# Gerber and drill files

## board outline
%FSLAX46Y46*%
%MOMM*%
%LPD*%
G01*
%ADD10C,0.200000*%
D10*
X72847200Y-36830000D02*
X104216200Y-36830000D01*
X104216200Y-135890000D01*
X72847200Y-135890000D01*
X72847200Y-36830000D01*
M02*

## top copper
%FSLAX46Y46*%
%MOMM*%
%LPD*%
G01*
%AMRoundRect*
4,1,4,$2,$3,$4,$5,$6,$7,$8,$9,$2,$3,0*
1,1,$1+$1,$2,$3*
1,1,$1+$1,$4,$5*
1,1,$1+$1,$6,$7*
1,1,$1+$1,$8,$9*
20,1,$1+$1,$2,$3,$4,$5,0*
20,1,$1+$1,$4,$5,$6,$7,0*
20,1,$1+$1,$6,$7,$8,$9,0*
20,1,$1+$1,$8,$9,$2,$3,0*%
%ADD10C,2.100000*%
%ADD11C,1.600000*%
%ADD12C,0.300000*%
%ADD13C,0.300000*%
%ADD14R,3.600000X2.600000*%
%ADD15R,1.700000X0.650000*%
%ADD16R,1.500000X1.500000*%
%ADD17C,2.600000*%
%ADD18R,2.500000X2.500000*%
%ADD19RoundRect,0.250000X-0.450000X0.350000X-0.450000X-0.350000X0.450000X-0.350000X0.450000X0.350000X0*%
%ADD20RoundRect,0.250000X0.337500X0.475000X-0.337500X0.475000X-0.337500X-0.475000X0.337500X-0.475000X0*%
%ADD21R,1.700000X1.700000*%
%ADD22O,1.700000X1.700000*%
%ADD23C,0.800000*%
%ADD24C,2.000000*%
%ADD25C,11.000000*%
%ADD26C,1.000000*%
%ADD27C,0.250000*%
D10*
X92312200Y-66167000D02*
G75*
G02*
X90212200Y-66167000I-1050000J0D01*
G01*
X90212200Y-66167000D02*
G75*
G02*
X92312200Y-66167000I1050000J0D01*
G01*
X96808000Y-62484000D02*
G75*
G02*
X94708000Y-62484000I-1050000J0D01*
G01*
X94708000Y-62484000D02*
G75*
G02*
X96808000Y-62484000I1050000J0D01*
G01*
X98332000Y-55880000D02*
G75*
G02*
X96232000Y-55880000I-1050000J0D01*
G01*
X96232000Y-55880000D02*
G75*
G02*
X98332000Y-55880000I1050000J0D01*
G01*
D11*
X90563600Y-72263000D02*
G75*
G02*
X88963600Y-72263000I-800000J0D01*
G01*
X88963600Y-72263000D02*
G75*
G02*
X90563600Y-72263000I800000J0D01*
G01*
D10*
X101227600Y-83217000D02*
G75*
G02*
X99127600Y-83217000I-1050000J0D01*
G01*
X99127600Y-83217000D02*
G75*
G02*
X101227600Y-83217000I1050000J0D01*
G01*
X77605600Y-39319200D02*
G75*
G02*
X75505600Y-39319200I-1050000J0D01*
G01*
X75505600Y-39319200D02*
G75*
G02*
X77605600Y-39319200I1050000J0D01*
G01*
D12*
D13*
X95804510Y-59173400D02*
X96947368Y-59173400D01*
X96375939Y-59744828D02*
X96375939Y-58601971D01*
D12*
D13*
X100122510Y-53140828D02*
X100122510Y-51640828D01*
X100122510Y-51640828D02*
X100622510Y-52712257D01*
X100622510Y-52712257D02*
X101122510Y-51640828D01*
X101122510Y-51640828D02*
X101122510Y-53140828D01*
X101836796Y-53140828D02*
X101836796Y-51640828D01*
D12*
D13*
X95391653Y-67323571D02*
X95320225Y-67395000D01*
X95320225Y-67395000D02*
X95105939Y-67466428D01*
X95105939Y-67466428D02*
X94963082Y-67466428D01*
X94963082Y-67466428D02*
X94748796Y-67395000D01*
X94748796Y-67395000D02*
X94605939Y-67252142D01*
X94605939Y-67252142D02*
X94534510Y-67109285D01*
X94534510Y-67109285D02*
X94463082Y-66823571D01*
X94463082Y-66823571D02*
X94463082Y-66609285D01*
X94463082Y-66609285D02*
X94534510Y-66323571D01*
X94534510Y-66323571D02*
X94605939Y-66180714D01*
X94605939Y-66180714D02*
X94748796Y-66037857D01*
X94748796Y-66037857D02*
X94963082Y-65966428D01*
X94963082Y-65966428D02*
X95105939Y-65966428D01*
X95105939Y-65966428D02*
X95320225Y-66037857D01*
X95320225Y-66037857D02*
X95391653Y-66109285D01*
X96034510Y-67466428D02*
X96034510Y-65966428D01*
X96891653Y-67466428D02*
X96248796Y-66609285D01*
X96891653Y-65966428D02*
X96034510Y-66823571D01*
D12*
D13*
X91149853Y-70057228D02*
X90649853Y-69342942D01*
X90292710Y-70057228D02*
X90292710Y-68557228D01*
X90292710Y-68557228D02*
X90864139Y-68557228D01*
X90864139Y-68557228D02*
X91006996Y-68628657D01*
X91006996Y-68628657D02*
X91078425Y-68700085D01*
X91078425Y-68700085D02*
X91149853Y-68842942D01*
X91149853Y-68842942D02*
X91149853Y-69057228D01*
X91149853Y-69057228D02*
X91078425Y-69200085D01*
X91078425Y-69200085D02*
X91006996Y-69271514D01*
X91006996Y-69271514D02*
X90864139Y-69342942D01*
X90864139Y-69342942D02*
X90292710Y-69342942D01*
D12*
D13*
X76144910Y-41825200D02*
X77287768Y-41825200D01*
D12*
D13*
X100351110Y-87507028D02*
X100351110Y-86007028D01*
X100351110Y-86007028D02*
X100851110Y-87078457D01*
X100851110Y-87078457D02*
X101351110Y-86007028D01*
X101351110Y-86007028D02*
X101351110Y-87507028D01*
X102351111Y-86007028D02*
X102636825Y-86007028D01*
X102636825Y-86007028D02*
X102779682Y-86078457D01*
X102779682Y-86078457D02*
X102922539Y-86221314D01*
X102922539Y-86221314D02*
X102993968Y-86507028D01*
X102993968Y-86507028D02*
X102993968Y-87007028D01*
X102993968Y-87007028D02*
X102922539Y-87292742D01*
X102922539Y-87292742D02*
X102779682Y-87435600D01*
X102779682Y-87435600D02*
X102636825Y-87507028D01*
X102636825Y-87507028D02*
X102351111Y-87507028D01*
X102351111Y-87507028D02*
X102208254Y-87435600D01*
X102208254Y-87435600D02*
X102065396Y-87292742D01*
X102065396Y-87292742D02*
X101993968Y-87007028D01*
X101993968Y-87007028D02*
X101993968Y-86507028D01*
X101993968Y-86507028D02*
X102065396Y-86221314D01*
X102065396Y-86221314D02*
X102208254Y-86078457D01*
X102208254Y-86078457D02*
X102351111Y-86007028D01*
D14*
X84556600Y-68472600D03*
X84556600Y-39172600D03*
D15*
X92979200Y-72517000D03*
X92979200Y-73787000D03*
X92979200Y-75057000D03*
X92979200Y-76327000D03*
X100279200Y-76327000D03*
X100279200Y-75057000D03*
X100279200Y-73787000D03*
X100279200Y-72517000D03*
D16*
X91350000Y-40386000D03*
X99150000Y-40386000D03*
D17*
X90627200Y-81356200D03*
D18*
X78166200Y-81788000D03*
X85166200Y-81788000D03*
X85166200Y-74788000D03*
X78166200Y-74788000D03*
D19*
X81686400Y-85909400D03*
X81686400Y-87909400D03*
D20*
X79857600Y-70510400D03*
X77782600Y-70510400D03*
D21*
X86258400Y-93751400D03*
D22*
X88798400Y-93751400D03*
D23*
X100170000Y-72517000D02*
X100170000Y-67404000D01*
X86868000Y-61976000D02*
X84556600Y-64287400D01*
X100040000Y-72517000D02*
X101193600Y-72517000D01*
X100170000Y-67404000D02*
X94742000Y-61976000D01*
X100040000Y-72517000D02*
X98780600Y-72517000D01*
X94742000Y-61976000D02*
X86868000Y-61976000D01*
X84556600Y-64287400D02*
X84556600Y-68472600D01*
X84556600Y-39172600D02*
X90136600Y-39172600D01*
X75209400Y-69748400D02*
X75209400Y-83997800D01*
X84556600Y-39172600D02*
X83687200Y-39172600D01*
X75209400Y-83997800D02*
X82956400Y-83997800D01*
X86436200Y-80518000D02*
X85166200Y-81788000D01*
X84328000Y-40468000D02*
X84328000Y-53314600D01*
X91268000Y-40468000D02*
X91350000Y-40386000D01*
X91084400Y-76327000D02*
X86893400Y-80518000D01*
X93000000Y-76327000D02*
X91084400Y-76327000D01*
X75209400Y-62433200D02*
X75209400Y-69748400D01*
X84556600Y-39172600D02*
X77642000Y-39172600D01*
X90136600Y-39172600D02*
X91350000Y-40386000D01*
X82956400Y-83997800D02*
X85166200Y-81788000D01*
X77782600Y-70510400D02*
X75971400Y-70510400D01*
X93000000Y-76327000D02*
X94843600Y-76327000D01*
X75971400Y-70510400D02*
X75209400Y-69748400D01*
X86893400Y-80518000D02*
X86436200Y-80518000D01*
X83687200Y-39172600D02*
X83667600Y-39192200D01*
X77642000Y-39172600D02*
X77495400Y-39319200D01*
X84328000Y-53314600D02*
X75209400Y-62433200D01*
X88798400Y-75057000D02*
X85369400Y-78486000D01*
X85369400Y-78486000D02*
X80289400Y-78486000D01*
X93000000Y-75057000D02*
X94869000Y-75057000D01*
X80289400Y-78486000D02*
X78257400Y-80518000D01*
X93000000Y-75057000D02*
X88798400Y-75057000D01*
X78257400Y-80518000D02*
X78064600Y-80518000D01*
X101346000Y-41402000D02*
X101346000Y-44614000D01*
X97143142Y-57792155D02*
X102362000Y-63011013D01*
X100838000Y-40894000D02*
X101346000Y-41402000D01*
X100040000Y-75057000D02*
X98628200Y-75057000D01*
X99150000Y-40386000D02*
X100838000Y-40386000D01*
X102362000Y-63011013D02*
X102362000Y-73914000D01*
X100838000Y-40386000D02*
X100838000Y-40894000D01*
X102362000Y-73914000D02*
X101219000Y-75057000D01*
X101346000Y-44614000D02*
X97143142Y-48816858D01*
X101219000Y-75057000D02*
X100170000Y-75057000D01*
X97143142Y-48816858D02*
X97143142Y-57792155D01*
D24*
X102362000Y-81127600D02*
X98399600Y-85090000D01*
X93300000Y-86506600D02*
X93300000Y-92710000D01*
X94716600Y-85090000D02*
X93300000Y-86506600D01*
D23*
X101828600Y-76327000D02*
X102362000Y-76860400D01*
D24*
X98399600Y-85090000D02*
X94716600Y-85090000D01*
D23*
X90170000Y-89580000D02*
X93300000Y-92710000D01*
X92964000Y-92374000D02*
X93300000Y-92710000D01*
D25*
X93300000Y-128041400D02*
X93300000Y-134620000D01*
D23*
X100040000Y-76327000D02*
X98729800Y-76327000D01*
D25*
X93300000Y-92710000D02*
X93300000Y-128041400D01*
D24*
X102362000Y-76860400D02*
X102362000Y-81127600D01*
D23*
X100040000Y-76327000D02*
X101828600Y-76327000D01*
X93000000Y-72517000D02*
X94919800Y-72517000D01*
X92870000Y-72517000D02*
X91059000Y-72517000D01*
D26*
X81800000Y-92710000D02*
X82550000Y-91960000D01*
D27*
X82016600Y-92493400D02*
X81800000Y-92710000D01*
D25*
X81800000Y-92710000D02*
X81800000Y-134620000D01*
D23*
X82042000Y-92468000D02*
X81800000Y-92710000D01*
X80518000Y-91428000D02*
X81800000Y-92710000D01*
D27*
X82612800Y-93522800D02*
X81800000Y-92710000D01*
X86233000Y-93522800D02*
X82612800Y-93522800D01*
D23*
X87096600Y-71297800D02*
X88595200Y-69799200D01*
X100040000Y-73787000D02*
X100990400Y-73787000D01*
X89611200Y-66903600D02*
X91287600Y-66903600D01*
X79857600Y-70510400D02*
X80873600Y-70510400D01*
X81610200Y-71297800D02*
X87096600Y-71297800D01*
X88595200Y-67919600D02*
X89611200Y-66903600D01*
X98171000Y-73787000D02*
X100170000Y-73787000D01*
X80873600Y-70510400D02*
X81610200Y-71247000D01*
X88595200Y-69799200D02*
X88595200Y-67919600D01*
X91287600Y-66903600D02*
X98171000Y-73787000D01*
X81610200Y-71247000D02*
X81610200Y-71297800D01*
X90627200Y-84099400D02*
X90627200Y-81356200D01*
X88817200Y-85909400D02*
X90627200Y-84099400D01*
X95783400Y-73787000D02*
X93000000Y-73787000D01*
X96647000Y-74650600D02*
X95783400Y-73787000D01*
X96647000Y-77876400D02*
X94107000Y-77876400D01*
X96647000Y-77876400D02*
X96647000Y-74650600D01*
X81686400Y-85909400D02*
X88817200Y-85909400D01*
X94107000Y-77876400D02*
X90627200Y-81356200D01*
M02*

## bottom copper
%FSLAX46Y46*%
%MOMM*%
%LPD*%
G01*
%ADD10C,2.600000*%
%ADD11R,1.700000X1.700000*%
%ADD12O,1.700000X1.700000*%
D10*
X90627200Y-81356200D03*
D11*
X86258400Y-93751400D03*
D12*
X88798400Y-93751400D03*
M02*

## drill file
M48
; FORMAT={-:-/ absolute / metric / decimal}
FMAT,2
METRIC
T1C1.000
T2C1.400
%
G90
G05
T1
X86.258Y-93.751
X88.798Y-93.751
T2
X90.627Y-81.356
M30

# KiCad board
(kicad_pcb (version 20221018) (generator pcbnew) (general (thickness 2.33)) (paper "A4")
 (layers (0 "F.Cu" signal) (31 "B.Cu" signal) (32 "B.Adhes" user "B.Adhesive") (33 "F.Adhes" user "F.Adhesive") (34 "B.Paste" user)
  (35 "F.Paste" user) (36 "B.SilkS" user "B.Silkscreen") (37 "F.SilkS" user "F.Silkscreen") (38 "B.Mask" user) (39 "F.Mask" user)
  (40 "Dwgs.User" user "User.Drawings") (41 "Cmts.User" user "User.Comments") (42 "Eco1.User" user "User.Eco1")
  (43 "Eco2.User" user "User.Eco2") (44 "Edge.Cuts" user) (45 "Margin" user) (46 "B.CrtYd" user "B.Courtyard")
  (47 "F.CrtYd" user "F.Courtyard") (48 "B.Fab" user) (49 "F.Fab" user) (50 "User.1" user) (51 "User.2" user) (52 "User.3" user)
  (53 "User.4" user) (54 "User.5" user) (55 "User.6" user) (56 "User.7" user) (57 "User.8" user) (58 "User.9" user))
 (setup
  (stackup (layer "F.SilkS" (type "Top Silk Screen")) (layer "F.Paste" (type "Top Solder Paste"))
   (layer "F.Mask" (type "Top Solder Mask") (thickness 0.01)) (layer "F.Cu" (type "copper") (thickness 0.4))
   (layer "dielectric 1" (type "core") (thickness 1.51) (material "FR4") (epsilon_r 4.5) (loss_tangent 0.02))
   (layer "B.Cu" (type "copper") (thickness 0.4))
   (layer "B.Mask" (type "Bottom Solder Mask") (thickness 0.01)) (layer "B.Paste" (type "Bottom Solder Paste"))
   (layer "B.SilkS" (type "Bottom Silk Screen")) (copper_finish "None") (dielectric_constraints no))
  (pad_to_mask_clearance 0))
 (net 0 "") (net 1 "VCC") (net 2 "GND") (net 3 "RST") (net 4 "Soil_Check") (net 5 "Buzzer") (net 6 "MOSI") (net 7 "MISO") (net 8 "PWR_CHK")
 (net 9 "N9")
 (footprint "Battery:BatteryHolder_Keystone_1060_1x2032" (layer "F.Cu") (at 84.5566 53.8226 90)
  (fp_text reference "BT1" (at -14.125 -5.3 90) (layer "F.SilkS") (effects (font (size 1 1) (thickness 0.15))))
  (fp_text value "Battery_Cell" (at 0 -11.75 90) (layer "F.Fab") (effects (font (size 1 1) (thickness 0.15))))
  (pad "1" smd rect (at -14.65 0 270) (size 2.6 3.6) (layers "F.Cu" "F.Paste" "F.Mask") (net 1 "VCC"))
  (pad "2" smd rect (at 14.65 0 270) (size 2.6 3.6) (layers "F.Cu" "F.Paste" "F.Mask") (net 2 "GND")))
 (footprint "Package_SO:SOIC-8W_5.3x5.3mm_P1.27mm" (layer "F.Cu") (at 96.6292 74.422)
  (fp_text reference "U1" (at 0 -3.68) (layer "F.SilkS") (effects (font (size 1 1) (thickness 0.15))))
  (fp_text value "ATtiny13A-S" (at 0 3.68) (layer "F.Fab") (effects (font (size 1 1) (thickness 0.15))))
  (pad "1" smd rect (at -3.65 -1.905) (size 1.7 0.65) (layers "F.Cu" "F.Paste" "F.Mask") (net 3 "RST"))
  (pad "2" smd rect (at -3.65 -0.635) (size 1.7 0.65) (layers "F.Cu" "F.Paste" "F.Mask") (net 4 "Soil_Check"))
  (pad "3" smd rect (at -3.65 0.635) (size 1.7 0.65) (layers "F.Cu" "F.Paste" "F.Mask") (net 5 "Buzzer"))
  (pad "4" smd rect (at -3.65 1.905) (size 1.7 0.65) (layers "F.Cu" "F.Paste" "F.Mask") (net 2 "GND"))
  (pad "5" smd rect (at 3.65 1.905) (size 1.7 0.65) (layers "F.Cu" "F.Paste" "F.Mask") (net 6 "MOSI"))
  (pad "6" smd rect (at 3.65 0.635) (size 1.7 0.65) (layers "F.Cu" "F.Paste" "F.Mask") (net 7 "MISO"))
  (pad "7" smd rect (at 3.65 -0.635) (size 1.7 0.65) (layers "F.Cu" "F.Paste" "F.Mask") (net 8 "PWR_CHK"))
  (pad "8" smd rect (at 3.65 -1.905) (size 1.7 0.65) (layers "F.Cu" "F.Paste" "F.Mask") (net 1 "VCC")))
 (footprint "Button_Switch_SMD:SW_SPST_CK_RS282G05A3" (layer "F.Cu") (at 95.25 40.386)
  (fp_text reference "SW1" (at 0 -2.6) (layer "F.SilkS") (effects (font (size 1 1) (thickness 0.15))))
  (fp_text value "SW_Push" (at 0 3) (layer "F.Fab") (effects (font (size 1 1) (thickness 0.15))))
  (pad "1" smd rect (at -3.9 0) (size 1.5 1.5) (layers "F.Cu" "F.Paste" "F.Mask") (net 2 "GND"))
  (pad "2" smd rect (at 3.9 0) (size 1.5 1.5) (layers "F.Cu" "F.Paste" "F.Mask") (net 7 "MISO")))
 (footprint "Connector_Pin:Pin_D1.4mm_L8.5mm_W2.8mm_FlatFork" (layer "F.Cu") (at 90.6272 81.3562)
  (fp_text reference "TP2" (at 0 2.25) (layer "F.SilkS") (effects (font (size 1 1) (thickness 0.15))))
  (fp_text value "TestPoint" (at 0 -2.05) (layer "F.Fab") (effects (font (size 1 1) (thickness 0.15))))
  (pad "1" thru_hole circle (at 0 0) (size 2.6 2.6) (drill 1.4) (layers "*.Cu" "*.Mask") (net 4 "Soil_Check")))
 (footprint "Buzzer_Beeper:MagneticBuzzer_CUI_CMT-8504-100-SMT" (layer "F.Cu") (at 81.6662 78.288 90)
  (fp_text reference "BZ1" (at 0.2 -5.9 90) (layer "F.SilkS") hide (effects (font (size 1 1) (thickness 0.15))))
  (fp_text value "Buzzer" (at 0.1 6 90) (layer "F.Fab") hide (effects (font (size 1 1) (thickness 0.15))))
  (pad "1" smd rect (at -3.5 -3.5) (size 2.5 2.5) (layers "F.Cu" "F.Paste" "F.Mask") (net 5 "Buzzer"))
  (pad "2" smd rect (at -3.5 3.5) (size 2.5 2.5) (layers "F.Cu" "F.Paste" "F.Mask") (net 2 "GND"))
  (pad "3" smd rect (at 3.5 3.5) (size 2.5 2.5) (layers "F.Cu" "F.Paste" "F.Mask"))
  (pad "4" smd rect (at 3.5 -3.5) (size 2.5 2.5) (layers "F.Cu" "F.Paste" "F.Mask")))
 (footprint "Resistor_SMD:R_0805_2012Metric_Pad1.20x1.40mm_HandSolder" (layer "F.Cu") (at 81.6864 86.9094 -90)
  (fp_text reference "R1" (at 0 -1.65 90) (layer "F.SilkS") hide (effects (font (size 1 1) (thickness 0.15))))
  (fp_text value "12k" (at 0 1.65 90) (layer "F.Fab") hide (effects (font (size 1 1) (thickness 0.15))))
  (pad "1" smd roundrect (at -1 0 270) (size 1.2 1.4) (layers "F.Cu" "F.Paste" "F.Mask") (roundrect_rratio 0.2083333333)
   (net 4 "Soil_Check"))
  (pad "2" smd roundrect (at 1 0 270) (size 1.2 1.4) (layers "F.Cu" "F.Paste" "F.Mask") (roundrect_rratio 0.2083333333) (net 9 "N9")))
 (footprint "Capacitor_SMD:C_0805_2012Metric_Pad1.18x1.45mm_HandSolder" (layer "F.Cu") (at 78.8201 70.5104 180)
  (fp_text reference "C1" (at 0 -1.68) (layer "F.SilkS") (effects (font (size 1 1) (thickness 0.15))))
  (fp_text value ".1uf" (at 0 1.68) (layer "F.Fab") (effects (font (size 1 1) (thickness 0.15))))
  (pad "1" smd roundrect (at -1.0375 0 180) (size 1.175 1.45) (layers "F.Cu" "F.Paste" "F.Mask") (roundrect_rratio 0.2127659574)
   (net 8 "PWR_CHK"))
  (pad "2" smd roundrect (at 1.0375 0 180) (size 1.175 1.45) (layers "F.Cu" "F.Paste" "F.Mask") (roundrect_rratio 0.2127659574)
   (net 2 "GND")))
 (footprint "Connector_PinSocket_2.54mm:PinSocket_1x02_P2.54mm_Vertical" (layer "F.Cu") (at 86.2584 93.7514 90)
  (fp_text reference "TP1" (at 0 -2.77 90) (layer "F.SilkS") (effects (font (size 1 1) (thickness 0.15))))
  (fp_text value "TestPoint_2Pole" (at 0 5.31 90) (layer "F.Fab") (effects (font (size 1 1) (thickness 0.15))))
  (pad "1" thru_hole rect (at 0 0 90) (size 1.7 1.7) (drill 1) (layers "*.Cu" "*.Mask") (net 9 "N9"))
  (pad "2" thru_hole oval (at 0 2.54 90) (size 1.7 1.7) (drill 1) (layers "*.Cu" "*.Mask") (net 6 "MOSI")))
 (gr_circle (center 91.2622 66.167) (end 93.2622 66.167) (stroke (width 0.2) (type solid)) (fill solid) (layer "F.Cu"))
 (gr_circle (center 95.758 62.484) (end 97.758 62.484) (stroke (width 0.2) (type solid)) (fill solid) (layer "F.Cu"))
 (gr_circle (center 97.282 55.88) (end 99.282 55.88) (stroke (width 0.2) (type solid)) (fill solid) (layer "F.Cu"))
 (gr_circle (center 89.7636 72.263) (end 91.2636 72.263) (stroke (width 0.2) (type solid)) (fill solid) (layer "F.Cu"))
 (gr_circle (center 100.1776 83.217) (end 102.1776 83.217) (stroke (width 0.2) (type solid)) (fill solid) (layer "F.Cu"))
 (gr_circle (center 76.5556 39.3192) (end 78.5556 39.3192) (stroke (width 0.2) (type solid)) (fill solid) (layer "F.Cu"))
 (gr_rect (start 72.8472 36.83) (end 104.2162 135.89) (stroke (width 0.2) (type default)) (fill none) (layer "Edge.Cuts"))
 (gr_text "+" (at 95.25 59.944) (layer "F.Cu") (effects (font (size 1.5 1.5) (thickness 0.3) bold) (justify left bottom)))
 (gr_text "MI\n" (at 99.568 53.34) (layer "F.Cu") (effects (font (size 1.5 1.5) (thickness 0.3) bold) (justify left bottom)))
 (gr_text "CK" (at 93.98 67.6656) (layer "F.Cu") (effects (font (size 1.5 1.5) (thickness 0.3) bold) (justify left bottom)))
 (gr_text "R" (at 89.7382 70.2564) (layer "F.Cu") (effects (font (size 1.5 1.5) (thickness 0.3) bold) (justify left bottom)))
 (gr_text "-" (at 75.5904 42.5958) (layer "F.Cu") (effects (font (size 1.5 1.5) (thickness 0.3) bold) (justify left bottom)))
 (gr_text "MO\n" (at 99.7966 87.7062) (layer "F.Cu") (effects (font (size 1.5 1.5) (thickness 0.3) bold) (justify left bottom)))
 (segment (start 100.17 72.517) (end 100.17 67.404) (width 0.8) (layer "F.Cu") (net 1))
 (segment (start 86.868 61.976) (end 84.5566 64.2874) (width 0.8) (layer "F.Cu") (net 1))
 (segment (start 100.04 72.517) (end 101.1936 72.517) (width 0.8) (layer "F.Cu") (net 1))
 (segment (start 100.17 67.404) (end 94.742 61.976) (width 0.8) (layer "F.Cu") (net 1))
 (segment (start 100.04 72.517) (end 98.7806 72.517) (width 0.8) (layer "F.Cu") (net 1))
 (segment (start 94.742 61.976) (end 86.868 61.976) (width 0.8) (layer "F.Cu") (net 1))
 (segment (start 84.5566 64.2874) (end 84.5566 68.4726) (width 0.8) (layer "F.Cu") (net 1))
 (segment (start 84.5566 39.1726) (end 90.1366 39.1726) (width 0.8) (layer "F.Cu") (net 2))
 (segment (start 75.2094 69.7484) (end 75.2094 83.9978) (width 0.8) (layer "F.Cu") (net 2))
 (segment (start 84.5566 39.1726) (end 83.6872 39.1726) (width 0.8) (layer "F.Cu") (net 2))
 (segment (start 75.2094 83.9978) (end 82.9564 83.9978) (width 0.8) (layer "F.Cu") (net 2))
 (segment (start 86.4362 80.518) (end 85.1662 81.788) (width 0.8) (layer "F.Cu") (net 2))
 (segment (start 84.328 40.468) (end 84.328 53.3146) (width 0.8) (layer "F.Cu") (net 2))
 (segment (start 91.268 40.468) (end 91.35 40.386) (width 0.8) (layer "F.Cu") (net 2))
 (segment (start 91.0844 76.327) (end 86.8934 80.518) (width 0.8) (layer "F.Cu") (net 2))
 (segment (start 93 76.327) (end 91.0844 76.327) (width 0.8) (layer "F.Cu") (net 2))
 (segment (start 75.2094 62.4332) (end 75.2094 69.7484) (width 0.8) (layer "F.Cu") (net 2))
 (segment (start 84.5566 39.1726) (end 77.642 39.1726) (width 0.8) (layer "F.Cu") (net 2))
 (segment (start 90.1366 39.1726) (end 91.35 40.386) (width 0.8) (layer "F.Cu") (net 2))
 (segment (start 82.9564 83.9978) (end 85.1662 81.788) (width 0.8) (layer "F.Cu") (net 2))
 (segment (start 77.7826 70.5104) (end 75.9714 70.5104) (width 0.8) (layer "F.Cu") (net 2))
 (segment (start 93 76.327) (end 94.8436 76.327) (width 0.8) (layer "F.Cu") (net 2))
 (segment (start 75.9714 70.5104) (end 75.2094 69.7484) (width 0.8) (layer "F.Cu") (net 2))
 (segment (start 86.8934 80.518) (end 86.4362 80.518) (width 0.8) (layer "F.Cu") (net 2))
 (segment (start 83.6872 39.1726) (end 83.6676 39.1922) (width 0.8) (layer "F.Cu") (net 2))
 (segment (start 77.642 39.1726) (end 77.4954 39.3192) (width 0.8) (layer "F.Cu") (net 2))
 (segment (start 84.328 53.3146) (end 75.2094 62.4332) (width 0.8) (layer "F.Cu") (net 2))
 (segment (start 88.7984 75.057) (end 85.3694 78.486) (width 0.8) (layer "F.Cu") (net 5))
 (segment (start 85.3694 78.486) (end 80.2894 78.486) (width 0.8) (layer "F.Cu") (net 5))
 (segment (start 93 75.057) (end 94.869 75.057) (width 0.8) (layer "F.Cu") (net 5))
 (segment (start 80.2894 78.486) (end 78.2574 80.518) (width 0.8) (layer "F.Cu") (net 5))
 (segment (start 93 75.057) (end 88.7984 75.057) (width 0.8) (layer "F.Cu") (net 5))
 (segment (start 78.2574 80.518) (end 78.0646 80.518) (width 0.8) (layer "F.Cu") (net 5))
 (segment (start 101.346 41.402) (end 101.346 44.614) (width 0.8) (layer "F.Cu") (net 7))
 (segment (start 97.143142 57.792155) (end 102.362 63.011013) (width 0.8) (layer "F.Cu") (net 7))
 (segment (start 100.838 40.894) (end 101.346 41.402) (width 0.8) (layer "F.Cu") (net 7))
 (segment (start 100.04 75.057) (end 98.6282 75.057) (width 0.8) (layer "F.Cu") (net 7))
 (segment (start 99.15 40.386) (end 100.838 40.386) (width 0.8) (layer "F.Cu") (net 7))
 (segment (start 102.362 63.011013) (end 102.362 73.914) (width 0.8) (layer "F.Cu") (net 7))
 (segment (start 100.838 40.386) (end 100.838 40.894) (width 0.8) (layer "F.Cu") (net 7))
 (segment (start 102.362 73.914) (end 101.219 75.057) (width 0.8) (layer "F.Cu") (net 7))
 (segment (start 101.346 44.614) (end 97.143142 48.816858) (width 0.8) (layer "F.Cu") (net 7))
 (segment (start 101.219 75.057) (end 100.17 75.057) (width 0.8) (layer "F.Cu") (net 7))
 (segment (start 97.143142 48.816858) (end 97.143142 57.792155) (width 0.8) (layer "F.Cu") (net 7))
 (segment (start 102.362 81.1276) (end 98.3996 85.09) (width 2) (layer "F.Cu") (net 6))
 (segment (start 93.3 86.5066) (end 93.3 92.71) (width 2) (layer "F.Cu") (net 6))
 (segment (start 94.7166 85.09) (end 93.3 86.5066) (width 2) (layer "F.Cu") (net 6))
 (segment (start 101.8286 76.327) (end 102.362 76.8604) (width 0.8) (layer "F.Cu") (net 6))
 (segment (start 98.3996 85.09) (end 94.7166 85.09) (width 2) (layer "F.Cu") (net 6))
 (segment (start 90.17 89.58) (end 93.3 92.71) (width 0.8) (layer "F.Cu") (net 6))
 (segment (start 92.964 92.374) (end 93.3 92.71) (width 0.8) (layer "F.Cu") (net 6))
 (segment (start 93.3 128.0414) (end 93.3 134.62) (width 11) (layer "F.Cu") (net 6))
 (segment (start 100.04 76.327) (end 98.7298 76.327) (width 0.8) (layer "F.Cu") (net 6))
 (segment (start 93.3 92.71) (end 93.3 128.0414) (width 11) (layer "F.Cu") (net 6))
 (segment (start 102.362 76.8604) (end 102.362 81.1276) (width 2) (layer "F.Cu") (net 6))
 (segment (start 100.04 76.327) (end 101.8286 76.327) (width 0.8) (layer "F.Cu") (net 6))
 (segment (start 93 72.517) (end 94.9198 72.517) (width 0.8) (layer "F.Cu") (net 3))
 (segment (start 92.87 72.517) (end 91.059 72.517) (width 0.8) (layer "F.Cu") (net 3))
 (segment (start 81.8 92.71) (end 82.55 91.96) (width 1) (layer "F.Cu") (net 9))
 (segment (start 82.0166 92.4934) (end 81.8 92.71) (width 0.25) (layer "F.Cu") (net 9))
 (segment (start 81.8 92.71) (end 81.8 134.62) (width 11) (layer "F.Cu") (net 9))
 (segment (start 82.042 92.468) (end 81.8 92.71) (width 0.8) (layer "F.Cu") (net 9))
 (segment (start 80.518 91.428) (end 81.8 92.71) (width 0.8) (layer "F.Cu") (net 9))
 (segment (start 82.6128 93.5228) (end 81.8 92.71) (width 0.25) (layer "F.Cu") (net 9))
 (segment (start 86.233 93.5228) (end 82.6128 93.5228) (width 0.25) (layer "F.Cu") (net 9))
 (segment (start 87.0966 71.2978) (end 88.5952 69.7992) (width 0.8) (layer "F.Cu") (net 8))
 (segment (start 100.04 73.787) (end 100.9904 73.787) (width 0.8) (layer "F.Cu") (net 8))
 (segment (start 89.6112 66.9036) (end 91.2876 66.9036) (width 0.8) (layer "F.Cu") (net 8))
 (segment (start 79.8576 70.5104) (end 80.8736 70.5104) (width 0.8) (layer "F.Cu") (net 8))
 (segment (start 81.6102 71.2978) (end 87.0966 71.2978) (width 0.8) (layer "F.Cu") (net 8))
 (segment (start 88.5952 67.9196) (end 89.6112 66.9036) (width 0.8) (layer "F.Cu") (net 8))
 (segment (start 98.171 73.787) (end 100.17 73.787) (width 0.8) (layer "F.Cu") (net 8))
 (segment (start 80.8736 70.5104) (end 81.6102 71.247) (width 0.8) (layer "F.Cu") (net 8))
 (segment (start 88.5952 69.7992) (end 88.5952 67.9196) (width 0.8) (layer "F.Cu") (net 8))
 (segment (start 91.2876 66.9036) (end 98.171 73.787) (width 0.8) (layer "F.Cu") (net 8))
 (segment (start 81.6102 71.247) (end 81.6102 71.2978) (width 0.8) (layer "F.Cu") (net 8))
 (segment (start 90.6272 84.0994) (end 90.6272 81.3562) (width 0.8) (layer "F.Cu") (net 4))
 (segment (start 88.8172 85.9094) (end 90.6272 84.0994) (width 0.8) (layer "F.Cu") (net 4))
 (segment (start 95.7834 73.787) (end 93 73.787) (width 0.8) (layer "F.Cu") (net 4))
 (segment (start 96.647 74.6506) (end 95.7834 73.787) (width 0.8) (layer "F.Cu") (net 4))
 (segment (start 96.647 77.8764) (end 94.107 77.8764) (width 0.8) (layer "F.Cu") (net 4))
 (segment (start 96.647 77.8764) (end 96.647 74.6506) (width 0.8) (layer "F.Cu") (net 4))
 (segment (start 81.6864 85.9094) (end 88.8172 85.9094) (width 0.8) (layer "F.Cu") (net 4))
 (segment (start 94.107 77.8764) (end 90.6272 81.3562) (width 0.8) (layer "F.Cu") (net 4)))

